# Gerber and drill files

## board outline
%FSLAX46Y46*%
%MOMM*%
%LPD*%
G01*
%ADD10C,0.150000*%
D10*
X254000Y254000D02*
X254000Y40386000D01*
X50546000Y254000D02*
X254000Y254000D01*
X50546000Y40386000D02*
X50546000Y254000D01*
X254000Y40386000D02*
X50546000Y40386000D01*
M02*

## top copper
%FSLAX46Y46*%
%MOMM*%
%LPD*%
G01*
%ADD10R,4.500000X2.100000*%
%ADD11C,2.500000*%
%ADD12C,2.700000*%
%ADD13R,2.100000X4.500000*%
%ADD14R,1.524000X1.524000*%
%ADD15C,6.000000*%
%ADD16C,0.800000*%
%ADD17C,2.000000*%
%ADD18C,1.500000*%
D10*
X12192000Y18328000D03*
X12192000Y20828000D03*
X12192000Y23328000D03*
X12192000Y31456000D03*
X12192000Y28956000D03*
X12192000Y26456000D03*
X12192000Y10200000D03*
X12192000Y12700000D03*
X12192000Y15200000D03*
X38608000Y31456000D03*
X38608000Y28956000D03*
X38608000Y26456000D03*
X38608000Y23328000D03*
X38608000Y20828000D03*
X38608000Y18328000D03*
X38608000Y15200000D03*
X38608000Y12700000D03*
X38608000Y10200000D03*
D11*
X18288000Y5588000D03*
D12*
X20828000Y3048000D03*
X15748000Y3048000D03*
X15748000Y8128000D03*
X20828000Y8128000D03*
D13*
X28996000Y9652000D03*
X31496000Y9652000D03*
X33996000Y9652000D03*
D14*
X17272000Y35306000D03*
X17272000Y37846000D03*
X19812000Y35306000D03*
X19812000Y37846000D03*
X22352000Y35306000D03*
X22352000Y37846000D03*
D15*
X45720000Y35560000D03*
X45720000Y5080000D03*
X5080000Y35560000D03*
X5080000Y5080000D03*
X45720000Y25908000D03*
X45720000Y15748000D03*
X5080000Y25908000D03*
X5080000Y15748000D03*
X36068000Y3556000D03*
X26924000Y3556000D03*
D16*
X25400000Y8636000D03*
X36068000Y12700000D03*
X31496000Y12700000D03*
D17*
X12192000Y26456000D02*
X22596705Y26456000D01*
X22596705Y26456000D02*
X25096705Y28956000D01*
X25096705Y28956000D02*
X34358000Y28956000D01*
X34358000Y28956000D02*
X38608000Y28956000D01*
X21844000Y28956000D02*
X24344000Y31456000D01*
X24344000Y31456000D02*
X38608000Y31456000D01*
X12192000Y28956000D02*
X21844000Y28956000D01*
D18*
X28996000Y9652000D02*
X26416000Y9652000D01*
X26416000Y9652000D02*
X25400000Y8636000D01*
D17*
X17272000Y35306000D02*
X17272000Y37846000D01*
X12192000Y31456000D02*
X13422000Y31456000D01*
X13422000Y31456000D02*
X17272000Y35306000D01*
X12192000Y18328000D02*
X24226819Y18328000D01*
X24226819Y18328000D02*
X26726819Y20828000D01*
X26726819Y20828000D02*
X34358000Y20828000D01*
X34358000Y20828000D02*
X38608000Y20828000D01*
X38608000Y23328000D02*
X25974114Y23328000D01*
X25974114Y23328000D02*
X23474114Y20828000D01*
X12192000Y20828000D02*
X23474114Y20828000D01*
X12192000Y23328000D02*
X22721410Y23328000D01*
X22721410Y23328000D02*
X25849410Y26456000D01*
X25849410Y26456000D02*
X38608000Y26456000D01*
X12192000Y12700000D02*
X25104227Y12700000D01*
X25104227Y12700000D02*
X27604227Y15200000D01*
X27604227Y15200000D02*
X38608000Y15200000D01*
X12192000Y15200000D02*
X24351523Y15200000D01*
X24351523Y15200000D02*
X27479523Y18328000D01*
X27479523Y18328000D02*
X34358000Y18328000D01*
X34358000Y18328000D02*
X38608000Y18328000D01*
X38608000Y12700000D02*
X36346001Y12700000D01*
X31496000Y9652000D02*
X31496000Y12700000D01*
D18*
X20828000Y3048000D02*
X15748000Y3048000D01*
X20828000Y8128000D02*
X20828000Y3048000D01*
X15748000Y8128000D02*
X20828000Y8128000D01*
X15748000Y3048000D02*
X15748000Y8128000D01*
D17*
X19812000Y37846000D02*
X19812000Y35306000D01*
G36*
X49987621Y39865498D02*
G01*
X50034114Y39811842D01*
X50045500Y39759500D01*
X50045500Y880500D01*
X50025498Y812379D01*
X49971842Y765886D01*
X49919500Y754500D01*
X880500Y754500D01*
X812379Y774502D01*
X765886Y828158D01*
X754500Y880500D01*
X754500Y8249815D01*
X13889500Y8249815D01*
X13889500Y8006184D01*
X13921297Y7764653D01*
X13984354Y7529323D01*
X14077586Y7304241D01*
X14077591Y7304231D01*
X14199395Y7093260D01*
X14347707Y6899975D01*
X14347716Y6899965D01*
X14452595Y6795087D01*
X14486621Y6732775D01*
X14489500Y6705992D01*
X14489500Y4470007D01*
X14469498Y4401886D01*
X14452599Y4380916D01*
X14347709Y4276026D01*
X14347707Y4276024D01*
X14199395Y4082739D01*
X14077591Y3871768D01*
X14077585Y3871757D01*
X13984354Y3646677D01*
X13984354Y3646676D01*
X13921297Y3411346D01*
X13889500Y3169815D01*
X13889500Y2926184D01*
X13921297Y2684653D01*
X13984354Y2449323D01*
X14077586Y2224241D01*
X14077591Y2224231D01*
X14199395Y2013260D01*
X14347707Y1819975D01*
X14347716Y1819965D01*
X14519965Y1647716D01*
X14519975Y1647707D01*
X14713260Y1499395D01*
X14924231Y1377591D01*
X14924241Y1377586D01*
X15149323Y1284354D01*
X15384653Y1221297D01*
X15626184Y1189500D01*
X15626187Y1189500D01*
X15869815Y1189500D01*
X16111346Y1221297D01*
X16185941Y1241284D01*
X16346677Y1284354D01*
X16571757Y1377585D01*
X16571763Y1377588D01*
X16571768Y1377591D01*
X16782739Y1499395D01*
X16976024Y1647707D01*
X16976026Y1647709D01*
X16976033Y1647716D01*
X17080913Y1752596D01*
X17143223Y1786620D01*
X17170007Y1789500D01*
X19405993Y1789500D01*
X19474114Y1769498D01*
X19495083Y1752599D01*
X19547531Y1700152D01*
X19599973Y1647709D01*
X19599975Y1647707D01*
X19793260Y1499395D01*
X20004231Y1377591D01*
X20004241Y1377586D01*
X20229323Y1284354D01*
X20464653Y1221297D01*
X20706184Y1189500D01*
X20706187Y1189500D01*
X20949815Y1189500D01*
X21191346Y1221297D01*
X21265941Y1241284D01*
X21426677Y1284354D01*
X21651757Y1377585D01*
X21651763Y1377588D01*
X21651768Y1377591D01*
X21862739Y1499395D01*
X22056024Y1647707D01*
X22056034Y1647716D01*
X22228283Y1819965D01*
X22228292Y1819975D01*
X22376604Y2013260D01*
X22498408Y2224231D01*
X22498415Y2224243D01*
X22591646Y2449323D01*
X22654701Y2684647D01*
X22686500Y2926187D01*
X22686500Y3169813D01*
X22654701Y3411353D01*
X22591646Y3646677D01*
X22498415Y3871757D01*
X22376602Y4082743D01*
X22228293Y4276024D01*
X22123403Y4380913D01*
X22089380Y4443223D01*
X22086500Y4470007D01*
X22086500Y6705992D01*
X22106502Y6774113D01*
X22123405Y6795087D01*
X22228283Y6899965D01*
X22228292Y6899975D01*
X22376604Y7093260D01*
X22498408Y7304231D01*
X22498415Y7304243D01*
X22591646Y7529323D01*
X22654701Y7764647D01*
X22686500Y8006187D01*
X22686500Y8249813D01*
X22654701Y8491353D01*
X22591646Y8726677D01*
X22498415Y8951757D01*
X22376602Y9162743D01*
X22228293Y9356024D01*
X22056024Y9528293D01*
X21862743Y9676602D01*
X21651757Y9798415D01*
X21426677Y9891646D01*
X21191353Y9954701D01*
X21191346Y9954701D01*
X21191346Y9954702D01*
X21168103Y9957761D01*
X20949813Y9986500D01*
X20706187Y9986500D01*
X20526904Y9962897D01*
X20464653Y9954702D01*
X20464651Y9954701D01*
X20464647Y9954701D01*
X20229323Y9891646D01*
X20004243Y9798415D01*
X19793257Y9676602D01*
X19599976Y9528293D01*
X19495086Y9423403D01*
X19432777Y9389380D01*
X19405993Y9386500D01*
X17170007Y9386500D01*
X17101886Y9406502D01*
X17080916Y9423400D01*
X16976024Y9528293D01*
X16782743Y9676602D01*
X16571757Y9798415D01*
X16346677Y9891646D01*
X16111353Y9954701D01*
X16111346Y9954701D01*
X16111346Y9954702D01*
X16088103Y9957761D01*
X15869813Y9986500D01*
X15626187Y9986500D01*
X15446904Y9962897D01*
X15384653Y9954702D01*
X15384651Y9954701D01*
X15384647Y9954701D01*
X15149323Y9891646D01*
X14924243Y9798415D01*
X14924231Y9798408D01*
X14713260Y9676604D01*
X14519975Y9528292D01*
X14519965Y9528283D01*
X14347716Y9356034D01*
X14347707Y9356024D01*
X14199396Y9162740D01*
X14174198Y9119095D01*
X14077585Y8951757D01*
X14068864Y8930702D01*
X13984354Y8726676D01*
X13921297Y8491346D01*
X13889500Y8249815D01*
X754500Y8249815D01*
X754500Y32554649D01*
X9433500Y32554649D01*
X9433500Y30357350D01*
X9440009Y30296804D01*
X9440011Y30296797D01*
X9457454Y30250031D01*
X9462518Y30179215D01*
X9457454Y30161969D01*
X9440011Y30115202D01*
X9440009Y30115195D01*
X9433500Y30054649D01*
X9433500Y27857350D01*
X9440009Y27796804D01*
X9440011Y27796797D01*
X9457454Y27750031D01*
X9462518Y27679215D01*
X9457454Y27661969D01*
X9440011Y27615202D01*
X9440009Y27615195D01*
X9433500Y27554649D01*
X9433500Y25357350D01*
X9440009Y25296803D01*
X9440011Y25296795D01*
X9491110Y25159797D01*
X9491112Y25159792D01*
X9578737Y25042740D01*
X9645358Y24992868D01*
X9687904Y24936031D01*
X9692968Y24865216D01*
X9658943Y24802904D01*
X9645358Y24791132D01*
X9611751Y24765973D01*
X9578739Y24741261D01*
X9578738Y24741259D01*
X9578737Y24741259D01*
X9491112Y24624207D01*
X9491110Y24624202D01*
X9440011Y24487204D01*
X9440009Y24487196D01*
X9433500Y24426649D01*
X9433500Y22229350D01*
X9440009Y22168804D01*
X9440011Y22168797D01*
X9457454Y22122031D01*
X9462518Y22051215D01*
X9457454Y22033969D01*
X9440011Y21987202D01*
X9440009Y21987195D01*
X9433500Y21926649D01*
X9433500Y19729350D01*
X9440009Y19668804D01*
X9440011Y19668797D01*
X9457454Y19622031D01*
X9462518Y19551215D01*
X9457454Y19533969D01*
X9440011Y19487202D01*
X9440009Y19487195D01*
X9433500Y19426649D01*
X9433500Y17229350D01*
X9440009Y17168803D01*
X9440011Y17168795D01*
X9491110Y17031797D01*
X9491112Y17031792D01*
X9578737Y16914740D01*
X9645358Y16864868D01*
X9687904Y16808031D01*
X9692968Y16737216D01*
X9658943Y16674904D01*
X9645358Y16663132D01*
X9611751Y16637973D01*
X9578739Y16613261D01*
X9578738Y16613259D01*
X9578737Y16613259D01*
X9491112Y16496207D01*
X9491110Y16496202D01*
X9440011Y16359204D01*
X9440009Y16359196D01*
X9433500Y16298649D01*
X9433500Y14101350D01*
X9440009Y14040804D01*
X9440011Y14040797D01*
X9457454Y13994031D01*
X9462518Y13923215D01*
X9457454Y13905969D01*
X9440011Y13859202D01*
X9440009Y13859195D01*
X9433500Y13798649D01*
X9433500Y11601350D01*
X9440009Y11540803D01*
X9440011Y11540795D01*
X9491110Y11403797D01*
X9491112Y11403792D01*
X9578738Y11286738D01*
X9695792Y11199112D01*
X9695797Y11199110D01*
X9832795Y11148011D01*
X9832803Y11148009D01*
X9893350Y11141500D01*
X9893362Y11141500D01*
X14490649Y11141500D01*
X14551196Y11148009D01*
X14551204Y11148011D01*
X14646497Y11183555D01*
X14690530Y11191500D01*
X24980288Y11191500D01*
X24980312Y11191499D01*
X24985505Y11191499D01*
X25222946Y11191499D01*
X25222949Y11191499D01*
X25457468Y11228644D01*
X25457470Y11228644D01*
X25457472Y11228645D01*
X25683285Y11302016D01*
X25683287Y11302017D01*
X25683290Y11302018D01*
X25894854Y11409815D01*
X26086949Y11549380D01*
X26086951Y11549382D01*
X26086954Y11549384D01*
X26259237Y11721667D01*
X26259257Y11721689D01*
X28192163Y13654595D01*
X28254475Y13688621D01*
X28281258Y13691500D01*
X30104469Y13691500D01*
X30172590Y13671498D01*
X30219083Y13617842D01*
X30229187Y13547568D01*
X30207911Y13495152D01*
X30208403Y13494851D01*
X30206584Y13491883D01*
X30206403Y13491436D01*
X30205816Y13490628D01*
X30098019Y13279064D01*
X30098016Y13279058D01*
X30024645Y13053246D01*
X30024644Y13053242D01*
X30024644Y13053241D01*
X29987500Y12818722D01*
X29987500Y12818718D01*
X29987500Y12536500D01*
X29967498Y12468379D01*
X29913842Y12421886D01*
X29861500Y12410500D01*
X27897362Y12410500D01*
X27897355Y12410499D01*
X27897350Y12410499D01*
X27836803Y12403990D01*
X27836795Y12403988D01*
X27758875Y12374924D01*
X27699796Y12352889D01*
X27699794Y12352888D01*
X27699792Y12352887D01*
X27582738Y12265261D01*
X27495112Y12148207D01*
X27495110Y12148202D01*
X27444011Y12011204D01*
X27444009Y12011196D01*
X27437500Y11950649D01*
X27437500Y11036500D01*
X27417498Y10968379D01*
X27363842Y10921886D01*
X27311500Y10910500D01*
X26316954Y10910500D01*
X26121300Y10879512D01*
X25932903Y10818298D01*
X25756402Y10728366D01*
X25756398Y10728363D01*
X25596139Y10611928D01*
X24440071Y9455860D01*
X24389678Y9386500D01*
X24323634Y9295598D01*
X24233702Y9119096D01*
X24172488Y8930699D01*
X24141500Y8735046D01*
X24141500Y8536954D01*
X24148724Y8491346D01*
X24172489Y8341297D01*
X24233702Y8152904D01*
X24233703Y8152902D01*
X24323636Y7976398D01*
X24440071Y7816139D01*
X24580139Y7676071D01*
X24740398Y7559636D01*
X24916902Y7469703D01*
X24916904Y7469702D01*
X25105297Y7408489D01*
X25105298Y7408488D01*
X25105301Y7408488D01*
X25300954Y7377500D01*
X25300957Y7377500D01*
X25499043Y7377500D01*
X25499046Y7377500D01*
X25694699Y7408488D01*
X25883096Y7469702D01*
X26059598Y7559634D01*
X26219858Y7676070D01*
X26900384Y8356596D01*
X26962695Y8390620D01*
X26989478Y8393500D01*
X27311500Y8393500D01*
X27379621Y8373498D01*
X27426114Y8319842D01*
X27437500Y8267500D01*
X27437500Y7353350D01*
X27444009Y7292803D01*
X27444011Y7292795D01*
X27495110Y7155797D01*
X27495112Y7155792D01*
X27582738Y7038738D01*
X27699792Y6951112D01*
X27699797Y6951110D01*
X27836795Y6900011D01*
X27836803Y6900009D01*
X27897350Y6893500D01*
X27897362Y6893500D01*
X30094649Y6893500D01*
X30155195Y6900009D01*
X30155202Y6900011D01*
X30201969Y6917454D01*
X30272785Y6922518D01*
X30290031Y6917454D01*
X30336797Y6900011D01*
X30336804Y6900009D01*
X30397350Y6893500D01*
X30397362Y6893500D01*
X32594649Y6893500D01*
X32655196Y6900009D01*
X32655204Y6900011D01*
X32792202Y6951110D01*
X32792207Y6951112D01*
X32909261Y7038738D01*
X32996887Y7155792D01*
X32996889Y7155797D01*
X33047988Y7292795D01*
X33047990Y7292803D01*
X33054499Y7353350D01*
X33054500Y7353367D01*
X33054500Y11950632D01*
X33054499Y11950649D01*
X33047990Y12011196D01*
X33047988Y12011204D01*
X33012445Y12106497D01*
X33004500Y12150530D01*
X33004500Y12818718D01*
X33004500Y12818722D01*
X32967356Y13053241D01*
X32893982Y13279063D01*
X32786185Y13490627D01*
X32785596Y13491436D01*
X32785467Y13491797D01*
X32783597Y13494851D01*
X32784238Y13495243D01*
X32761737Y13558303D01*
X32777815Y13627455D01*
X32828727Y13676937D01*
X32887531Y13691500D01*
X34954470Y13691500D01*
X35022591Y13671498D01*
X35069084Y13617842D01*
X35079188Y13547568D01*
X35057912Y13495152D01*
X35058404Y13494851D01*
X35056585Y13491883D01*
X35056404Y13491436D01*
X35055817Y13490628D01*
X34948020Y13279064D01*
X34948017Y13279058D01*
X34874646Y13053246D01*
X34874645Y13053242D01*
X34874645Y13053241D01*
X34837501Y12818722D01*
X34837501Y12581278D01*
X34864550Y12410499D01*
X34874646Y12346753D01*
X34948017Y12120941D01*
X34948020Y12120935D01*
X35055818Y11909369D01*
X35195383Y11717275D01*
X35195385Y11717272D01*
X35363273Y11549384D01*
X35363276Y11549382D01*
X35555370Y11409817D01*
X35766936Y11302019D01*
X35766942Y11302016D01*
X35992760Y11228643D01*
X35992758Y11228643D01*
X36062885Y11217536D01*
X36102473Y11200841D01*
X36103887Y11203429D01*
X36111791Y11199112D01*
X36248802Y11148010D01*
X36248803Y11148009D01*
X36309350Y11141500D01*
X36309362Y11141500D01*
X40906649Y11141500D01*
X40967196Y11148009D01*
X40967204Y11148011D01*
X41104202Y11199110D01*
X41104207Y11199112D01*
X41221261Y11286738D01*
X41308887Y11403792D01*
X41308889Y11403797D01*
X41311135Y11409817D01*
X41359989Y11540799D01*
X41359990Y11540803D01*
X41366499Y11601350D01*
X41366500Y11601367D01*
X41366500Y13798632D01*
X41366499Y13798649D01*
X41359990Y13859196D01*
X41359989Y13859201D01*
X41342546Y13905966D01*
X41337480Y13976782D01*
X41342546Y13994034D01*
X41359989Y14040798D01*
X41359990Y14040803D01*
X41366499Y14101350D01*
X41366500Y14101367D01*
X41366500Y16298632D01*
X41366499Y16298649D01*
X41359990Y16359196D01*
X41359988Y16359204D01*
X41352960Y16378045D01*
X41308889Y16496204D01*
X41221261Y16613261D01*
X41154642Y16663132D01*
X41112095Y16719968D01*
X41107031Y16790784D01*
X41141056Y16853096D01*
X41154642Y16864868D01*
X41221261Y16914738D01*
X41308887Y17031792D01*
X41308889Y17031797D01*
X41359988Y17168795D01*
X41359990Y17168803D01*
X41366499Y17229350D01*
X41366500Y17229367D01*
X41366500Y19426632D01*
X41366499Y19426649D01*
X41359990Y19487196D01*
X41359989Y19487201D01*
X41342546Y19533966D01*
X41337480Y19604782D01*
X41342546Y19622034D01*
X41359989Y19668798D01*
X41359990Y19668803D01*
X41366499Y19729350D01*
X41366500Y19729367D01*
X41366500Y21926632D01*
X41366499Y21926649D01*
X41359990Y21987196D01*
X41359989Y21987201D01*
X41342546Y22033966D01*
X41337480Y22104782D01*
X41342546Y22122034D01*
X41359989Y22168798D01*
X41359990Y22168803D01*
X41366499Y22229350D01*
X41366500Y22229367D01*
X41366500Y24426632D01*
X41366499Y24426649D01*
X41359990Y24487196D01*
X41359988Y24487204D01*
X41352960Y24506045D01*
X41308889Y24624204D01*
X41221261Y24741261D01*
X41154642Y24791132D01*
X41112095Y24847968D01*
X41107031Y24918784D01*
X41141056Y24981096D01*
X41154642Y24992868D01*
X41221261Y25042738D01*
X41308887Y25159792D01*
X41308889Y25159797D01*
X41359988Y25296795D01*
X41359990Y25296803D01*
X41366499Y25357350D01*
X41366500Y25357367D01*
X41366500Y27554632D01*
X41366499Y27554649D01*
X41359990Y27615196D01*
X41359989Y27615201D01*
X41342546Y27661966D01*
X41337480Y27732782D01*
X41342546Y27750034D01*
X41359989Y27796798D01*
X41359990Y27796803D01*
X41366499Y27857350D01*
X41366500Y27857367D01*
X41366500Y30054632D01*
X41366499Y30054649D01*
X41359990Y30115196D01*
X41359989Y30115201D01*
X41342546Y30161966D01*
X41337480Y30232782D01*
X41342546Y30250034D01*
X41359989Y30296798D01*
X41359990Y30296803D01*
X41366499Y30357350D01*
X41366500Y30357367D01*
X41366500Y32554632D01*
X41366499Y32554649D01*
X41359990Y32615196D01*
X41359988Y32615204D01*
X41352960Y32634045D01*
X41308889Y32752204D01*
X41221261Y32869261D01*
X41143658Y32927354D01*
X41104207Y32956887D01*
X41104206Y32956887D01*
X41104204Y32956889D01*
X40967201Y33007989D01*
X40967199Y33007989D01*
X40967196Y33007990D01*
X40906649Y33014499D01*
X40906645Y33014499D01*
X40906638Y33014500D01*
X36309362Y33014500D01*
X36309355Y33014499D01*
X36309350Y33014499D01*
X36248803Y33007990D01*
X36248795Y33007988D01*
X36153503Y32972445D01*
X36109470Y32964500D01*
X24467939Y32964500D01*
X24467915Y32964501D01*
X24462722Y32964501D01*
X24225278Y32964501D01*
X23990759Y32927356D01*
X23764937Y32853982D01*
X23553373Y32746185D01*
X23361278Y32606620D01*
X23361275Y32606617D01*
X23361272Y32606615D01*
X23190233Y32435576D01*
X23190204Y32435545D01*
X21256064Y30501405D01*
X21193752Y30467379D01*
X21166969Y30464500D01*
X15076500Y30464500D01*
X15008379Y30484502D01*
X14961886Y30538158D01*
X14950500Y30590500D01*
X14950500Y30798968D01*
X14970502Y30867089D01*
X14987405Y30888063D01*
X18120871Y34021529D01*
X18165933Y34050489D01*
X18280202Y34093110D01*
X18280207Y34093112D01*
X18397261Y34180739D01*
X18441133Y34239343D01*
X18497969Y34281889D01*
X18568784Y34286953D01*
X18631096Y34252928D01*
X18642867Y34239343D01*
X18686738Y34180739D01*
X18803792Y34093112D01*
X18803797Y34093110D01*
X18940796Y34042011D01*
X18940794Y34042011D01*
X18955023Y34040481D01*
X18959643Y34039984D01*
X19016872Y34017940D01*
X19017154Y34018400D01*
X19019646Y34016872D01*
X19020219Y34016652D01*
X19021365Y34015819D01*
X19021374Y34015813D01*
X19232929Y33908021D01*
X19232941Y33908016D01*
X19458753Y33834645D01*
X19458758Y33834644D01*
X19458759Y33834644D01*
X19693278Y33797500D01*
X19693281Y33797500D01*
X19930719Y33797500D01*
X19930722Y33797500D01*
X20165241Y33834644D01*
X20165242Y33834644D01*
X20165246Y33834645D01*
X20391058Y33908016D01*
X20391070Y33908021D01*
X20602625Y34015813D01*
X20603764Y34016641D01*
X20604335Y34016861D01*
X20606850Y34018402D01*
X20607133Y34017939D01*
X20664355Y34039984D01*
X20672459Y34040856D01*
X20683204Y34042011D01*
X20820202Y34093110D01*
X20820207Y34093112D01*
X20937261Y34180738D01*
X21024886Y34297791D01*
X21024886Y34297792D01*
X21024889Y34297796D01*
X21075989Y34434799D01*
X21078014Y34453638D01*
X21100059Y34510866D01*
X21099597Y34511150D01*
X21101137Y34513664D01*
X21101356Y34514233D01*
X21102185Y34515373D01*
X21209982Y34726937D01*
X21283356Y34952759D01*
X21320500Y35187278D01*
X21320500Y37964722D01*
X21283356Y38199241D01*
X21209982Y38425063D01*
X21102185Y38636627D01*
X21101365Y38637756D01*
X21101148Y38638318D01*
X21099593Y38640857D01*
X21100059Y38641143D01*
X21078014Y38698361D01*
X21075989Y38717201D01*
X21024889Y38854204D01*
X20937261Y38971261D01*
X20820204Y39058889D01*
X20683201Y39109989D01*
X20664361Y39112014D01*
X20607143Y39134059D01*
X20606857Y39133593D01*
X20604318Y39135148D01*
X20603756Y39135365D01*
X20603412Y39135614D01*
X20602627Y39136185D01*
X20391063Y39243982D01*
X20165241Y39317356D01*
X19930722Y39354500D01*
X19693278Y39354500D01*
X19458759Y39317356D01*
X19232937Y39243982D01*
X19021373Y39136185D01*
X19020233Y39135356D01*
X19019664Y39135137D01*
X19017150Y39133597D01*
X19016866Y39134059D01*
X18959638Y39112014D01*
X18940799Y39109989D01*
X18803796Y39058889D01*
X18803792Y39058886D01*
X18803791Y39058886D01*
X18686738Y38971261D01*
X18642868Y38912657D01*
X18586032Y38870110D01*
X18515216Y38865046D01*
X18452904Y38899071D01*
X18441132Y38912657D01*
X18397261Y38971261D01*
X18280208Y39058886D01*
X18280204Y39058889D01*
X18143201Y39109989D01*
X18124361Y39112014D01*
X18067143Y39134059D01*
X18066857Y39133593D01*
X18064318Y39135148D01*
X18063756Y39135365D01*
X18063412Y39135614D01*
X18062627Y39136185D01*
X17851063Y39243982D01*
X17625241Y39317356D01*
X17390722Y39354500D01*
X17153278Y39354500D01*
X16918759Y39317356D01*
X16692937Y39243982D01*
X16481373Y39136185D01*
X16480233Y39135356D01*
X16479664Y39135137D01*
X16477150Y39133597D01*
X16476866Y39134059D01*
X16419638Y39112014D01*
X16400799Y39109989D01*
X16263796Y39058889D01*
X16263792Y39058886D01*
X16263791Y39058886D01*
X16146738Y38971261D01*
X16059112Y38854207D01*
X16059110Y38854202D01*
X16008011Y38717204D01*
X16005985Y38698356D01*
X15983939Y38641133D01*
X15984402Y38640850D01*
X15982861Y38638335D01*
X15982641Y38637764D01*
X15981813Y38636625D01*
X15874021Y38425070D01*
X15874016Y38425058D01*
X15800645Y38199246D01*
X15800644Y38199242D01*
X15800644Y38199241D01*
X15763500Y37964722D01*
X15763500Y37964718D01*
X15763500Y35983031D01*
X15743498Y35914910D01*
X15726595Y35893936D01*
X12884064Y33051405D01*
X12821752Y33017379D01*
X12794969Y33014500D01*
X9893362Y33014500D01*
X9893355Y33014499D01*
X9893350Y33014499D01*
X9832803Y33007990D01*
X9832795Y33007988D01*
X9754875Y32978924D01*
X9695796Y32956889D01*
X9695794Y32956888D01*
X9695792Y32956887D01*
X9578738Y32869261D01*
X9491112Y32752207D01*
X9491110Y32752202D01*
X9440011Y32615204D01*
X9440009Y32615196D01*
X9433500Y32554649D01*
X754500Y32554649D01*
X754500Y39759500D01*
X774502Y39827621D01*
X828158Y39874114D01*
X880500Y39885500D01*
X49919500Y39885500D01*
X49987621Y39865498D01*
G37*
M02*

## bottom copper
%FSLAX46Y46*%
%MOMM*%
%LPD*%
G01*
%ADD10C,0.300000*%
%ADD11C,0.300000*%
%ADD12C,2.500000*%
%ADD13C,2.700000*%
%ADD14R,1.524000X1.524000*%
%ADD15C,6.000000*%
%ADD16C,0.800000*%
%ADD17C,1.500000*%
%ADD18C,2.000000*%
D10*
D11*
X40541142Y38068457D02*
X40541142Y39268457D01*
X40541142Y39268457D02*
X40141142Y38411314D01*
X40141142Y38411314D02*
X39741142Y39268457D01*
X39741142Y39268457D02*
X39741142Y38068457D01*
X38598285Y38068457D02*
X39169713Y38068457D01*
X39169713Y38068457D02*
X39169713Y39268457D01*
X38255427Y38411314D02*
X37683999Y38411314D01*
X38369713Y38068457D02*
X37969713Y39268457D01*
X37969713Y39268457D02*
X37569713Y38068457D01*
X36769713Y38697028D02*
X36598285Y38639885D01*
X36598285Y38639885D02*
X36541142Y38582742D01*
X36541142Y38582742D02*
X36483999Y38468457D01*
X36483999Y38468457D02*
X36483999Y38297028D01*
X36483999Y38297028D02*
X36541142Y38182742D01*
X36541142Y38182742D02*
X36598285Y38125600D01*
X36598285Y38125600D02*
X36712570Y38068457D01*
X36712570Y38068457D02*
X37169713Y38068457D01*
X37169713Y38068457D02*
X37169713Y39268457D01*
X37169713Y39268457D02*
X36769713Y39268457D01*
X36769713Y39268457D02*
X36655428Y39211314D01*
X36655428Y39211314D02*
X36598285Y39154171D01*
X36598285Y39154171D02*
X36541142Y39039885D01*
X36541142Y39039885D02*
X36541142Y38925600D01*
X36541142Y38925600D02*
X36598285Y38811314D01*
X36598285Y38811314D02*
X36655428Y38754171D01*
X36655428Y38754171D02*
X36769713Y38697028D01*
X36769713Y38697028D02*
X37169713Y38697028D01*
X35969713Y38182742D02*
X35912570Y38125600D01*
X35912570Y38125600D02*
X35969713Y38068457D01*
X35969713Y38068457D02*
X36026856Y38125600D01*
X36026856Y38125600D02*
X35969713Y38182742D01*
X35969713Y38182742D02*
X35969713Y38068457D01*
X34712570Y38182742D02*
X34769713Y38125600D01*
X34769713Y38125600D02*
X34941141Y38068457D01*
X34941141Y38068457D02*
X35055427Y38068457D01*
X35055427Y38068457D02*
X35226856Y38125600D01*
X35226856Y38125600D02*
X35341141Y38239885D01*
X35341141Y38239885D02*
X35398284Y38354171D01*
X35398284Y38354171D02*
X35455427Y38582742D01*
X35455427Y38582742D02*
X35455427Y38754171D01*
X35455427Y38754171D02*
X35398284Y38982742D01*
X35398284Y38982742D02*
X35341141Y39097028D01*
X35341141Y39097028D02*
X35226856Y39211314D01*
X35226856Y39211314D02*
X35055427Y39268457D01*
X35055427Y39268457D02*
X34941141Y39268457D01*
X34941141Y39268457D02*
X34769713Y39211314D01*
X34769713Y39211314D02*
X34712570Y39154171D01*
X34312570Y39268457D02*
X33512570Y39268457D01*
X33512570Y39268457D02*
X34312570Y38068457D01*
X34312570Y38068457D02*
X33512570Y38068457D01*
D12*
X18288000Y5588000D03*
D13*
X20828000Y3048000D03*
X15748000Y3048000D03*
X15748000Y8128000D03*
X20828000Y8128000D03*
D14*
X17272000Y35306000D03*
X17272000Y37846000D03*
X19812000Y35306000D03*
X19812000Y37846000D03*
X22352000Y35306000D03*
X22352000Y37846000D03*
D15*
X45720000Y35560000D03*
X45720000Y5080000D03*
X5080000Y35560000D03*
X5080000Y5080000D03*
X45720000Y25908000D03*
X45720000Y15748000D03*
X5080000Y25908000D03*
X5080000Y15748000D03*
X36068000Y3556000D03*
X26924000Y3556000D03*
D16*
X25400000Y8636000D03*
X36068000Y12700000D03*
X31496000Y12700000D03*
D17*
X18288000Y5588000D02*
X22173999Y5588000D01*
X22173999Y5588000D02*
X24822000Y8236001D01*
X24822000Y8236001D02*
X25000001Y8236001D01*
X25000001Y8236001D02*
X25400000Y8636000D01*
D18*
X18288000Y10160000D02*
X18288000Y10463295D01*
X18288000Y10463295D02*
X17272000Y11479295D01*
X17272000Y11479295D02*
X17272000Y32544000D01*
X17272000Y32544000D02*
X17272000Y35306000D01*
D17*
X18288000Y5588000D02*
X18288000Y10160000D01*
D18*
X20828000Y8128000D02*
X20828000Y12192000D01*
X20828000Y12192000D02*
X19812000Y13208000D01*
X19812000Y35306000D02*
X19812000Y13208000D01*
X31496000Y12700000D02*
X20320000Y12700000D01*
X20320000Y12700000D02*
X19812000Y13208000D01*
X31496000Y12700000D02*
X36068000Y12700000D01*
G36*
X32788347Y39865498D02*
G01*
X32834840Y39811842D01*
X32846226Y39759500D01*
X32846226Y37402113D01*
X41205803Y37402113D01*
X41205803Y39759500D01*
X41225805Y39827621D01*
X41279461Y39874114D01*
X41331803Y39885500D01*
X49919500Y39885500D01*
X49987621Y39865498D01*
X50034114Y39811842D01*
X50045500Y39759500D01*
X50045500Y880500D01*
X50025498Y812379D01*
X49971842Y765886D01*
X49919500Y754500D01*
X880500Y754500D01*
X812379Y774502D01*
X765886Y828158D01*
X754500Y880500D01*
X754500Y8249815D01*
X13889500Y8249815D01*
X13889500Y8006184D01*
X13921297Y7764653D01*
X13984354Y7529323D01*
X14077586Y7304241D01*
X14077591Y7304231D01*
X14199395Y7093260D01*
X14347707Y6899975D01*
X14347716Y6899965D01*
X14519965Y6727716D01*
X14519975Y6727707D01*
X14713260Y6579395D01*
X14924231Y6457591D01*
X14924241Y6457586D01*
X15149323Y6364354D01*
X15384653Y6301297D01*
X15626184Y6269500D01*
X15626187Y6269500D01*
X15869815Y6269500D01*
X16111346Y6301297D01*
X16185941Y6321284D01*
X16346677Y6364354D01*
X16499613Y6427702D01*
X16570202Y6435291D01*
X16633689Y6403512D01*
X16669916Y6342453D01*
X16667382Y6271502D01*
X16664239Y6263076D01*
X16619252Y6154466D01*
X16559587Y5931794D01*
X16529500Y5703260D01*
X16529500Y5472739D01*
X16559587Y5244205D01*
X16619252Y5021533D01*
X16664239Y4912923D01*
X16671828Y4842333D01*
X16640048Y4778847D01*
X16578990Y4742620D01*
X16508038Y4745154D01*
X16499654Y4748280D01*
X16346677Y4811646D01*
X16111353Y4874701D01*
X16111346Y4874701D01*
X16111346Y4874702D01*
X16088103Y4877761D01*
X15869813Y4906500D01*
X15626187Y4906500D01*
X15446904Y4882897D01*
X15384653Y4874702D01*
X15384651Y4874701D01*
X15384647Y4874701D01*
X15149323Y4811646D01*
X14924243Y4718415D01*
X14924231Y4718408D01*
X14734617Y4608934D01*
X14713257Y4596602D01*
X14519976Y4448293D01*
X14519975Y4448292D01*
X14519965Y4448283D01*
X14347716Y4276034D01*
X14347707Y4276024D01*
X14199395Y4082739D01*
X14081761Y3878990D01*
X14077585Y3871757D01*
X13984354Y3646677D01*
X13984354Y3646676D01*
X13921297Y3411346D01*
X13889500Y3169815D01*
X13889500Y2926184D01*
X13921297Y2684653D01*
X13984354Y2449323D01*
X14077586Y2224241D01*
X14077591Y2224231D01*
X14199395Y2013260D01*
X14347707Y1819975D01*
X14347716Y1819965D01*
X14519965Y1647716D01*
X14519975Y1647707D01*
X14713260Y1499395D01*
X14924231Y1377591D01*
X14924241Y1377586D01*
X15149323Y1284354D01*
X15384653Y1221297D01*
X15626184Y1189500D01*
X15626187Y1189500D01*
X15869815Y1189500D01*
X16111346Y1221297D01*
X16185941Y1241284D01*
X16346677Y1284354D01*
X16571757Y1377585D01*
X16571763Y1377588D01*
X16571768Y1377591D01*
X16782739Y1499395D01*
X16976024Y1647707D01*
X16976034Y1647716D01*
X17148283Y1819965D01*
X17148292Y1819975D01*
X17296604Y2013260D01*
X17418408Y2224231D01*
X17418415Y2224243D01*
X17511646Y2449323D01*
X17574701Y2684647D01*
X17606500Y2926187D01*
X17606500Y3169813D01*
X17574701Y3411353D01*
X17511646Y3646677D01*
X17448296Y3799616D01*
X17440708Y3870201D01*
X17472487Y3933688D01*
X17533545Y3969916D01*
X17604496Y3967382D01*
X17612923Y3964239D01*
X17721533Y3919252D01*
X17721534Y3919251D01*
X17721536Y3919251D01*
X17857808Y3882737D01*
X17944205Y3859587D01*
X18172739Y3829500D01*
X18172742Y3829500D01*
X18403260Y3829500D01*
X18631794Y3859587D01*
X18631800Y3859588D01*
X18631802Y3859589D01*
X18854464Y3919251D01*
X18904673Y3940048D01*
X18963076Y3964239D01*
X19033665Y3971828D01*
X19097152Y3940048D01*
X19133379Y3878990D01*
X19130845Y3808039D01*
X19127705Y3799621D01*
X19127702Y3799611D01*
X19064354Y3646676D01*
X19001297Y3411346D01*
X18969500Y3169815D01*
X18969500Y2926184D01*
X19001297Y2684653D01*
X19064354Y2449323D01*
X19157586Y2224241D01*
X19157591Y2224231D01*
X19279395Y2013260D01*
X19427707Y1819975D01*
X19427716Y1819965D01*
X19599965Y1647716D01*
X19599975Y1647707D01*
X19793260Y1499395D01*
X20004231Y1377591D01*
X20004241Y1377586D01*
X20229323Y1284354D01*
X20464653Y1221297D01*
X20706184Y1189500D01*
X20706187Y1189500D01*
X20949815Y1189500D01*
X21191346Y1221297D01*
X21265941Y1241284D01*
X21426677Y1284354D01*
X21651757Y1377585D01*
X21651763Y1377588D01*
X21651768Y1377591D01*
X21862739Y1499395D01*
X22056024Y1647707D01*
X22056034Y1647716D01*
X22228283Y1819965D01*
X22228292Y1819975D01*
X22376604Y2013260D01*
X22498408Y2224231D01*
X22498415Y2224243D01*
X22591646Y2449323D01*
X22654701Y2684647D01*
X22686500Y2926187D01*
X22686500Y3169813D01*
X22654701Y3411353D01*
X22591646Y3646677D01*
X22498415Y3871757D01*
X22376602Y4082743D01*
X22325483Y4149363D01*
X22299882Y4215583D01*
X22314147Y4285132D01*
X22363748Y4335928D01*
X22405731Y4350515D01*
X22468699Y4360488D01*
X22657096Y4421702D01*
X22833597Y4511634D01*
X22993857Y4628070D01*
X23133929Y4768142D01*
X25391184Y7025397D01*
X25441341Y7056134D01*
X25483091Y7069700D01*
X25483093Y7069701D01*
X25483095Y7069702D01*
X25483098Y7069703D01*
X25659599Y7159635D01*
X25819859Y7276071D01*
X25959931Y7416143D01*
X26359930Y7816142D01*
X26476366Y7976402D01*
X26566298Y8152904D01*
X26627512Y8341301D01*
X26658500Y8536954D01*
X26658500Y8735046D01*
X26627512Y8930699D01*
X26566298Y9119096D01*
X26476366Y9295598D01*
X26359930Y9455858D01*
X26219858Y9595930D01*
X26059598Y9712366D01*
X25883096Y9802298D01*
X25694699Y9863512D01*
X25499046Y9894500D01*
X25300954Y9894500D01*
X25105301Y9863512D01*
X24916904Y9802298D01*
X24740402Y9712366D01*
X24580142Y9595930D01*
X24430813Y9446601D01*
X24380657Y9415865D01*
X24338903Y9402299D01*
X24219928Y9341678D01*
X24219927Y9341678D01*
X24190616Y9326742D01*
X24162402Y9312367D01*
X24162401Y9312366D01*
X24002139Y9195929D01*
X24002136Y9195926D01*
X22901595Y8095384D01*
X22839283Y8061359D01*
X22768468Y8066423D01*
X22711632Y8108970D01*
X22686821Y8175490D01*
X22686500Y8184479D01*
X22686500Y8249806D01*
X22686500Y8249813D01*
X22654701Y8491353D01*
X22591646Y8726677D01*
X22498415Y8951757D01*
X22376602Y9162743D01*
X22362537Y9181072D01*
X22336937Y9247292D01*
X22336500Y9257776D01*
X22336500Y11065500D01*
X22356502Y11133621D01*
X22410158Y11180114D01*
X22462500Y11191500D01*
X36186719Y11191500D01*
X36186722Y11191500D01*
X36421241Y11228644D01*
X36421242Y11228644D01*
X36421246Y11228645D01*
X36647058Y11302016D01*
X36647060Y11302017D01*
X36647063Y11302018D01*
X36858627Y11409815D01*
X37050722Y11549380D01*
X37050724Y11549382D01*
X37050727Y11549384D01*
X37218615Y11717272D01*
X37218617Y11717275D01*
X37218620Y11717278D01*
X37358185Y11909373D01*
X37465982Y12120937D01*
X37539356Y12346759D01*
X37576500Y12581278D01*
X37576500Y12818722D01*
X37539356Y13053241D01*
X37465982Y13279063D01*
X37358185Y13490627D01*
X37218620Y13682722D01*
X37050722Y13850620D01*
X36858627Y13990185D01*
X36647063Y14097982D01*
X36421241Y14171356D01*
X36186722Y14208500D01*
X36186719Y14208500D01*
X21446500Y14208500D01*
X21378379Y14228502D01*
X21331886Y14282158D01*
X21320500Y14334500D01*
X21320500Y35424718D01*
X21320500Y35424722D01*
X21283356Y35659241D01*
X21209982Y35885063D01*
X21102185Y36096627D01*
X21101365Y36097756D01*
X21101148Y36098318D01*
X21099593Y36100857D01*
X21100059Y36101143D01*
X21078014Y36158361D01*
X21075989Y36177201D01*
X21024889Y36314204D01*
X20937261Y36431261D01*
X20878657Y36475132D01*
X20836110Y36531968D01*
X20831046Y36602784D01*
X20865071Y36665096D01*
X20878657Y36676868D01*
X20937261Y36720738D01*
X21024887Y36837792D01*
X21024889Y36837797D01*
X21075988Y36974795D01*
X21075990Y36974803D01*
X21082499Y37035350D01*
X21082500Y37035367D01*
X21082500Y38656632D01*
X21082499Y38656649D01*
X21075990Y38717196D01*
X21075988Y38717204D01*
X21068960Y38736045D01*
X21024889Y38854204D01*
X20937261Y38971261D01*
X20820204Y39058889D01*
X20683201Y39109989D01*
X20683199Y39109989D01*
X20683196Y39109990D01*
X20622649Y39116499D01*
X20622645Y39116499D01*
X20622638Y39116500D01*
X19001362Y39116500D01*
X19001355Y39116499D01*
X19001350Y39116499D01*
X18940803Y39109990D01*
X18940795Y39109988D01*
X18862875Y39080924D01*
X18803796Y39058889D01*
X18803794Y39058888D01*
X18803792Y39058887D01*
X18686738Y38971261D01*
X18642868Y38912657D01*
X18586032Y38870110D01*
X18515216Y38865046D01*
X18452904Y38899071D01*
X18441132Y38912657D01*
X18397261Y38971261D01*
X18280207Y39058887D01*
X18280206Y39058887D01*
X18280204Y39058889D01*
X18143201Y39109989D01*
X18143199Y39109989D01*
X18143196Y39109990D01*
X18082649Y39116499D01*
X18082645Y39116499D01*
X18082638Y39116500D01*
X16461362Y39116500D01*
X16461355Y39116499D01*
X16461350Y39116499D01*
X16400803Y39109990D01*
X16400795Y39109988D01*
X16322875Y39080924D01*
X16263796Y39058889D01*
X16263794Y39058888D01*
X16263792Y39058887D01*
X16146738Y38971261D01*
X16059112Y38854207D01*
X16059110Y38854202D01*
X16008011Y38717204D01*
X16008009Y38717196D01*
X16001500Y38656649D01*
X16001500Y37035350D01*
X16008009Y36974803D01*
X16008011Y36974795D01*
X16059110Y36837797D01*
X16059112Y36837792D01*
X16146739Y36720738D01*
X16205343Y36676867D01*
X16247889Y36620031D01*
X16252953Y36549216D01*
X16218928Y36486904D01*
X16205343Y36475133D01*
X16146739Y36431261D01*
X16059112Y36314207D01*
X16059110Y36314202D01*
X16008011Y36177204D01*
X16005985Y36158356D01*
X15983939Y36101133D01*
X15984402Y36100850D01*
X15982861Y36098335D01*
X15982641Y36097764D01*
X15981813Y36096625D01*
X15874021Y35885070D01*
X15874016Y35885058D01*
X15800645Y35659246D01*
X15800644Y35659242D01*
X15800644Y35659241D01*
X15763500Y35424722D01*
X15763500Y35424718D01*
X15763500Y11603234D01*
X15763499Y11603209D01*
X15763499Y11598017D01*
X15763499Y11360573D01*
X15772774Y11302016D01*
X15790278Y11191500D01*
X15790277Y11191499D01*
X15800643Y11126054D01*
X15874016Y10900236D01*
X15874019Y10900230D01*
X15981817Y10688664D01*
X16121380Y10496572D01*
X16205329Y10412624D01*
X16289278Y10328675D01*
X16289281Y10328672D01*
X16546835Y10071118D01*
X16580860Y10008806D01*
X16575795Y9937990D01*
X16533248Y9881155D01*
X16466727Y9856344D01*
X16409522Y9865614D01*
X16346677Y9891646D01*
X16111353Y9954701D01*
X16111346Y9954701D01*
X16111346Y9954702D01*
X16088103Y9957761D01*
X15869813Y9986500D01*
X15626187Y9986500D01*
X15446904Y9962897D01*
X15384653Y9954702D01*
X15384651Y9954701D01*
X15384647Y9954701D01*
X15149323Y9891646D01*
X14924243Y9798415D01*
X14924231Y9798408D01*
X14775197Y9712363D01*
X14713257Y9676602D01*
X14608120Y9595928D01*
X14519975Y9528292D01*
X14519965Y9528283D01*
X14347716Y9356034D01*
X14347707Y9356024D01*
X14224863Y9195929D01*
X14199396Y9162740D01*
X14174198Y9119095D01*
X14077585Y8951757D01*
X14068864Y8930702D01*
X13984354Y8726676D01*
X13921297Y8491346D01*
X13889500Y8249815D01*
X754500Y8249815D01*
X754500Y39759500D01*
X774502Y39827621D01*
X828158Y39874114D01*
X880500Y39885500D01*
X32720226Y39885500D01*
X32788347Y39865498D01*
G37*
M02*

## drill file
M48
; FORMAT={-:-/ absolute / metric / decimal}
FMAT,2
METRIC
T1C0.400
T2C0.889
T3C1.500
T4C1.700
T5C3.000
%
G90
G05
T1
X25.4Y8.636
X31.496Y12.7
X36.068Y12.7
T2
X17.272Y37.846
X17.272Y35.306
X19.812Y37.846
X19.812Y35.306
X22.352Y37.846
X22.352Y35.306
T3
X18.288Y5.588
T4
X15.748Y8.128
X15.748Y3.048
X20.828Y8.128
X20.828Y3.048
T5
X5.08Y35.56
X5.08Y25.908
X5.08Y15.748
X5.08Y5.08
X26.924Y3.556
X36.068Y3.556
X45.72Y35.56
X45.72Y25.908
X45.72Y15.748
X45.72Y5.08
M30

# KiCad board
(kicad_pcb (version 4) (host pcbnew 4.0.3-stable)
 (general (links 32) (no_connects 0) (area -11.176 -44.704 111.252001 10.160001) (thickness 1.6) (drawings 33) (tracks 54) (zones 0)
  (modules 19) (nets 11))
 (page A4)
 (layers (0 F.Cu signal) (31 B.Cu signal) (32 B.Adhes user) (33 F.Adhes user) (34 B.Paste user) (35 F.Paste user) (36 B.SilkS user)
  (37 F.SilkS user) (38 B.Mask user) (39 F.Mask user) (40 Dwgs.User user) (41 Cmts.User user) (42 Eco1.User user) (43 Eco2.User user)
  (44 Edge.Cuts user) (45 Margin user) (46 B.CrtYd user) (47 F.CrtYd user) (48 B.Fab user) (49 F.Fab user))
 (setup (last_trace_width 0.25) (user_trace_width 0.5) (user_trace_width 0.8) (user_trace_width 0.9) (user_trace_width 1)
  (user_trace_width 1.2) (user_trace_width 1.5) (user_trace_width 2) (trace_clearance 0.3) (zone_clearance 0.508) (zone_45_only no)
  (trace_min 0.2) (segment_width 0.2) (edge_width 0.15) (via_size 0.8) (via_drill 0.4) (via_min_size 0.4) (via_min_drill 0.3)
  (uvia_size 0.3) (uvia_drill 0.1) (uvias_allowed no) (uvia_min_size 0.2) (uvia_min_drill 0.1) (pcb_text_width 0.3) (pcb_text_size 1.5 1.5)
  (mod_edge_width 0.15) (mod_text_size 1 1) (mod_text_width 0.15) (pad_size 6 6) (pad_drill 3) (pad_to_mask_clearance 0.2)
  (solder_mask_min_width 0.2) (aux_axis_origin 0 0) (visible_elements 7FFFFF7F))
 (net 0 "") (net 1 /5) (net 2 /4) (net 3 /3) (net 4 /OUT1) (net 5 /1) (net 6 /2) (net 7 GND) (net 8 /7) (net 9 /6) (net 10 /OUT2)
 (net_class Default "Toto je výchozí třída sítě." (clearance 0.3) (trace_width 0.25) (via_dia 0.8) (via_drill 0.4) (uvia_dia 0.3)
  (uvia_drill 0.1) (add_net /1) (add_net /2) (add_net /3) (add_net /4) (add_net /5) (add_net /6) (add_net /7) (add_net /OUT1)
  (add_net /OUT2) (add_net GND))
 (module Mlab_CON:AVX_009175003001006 (layer F.Cu) (at 12.192 -20.828 90)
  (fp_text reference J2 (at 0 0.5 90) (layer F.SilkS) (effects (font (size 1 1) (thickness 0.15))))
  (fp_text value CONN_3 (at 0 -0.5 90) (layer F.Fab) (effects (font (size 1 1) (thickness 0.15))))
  (pad 1 smd rect (at -2.5 0 90) (size 2.1 4.5) (layers F.Cu F.Paste F.Mask) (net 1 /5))
  (pad 2 smd rect (at 0 0 90) (size 2.1 4.5) (layers F.Cu F.Paste F.Mask) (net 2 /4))
  (pad 3 smd rect (at 2.5 0 90) (size 2.1 4.5) (layers F.Cu F.Paste F.Mask) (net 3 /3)))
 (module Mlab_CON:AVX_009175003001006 (layer F.Cu) (at 12.192 -28.956 270)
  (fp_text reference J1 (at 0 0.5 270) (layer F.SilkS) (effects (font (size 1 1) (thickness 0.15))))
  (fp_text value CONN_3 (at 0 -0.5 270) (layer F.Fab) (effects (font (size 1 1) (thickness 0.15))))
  (pad 1 smd rect (at -2.5 0 270) (size 2.1 4.5) (layers F.Cu F.Paste F.Mask) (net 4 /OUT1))
  (pad 2 smd rect (at 0 0 270) (size 2.1 4.5) (layers F.Cu F.Paste F.Mask) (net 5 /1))
  (pad 3 smd rect (at 2.5 0 270) (size 2.1 4.5) (layers F.Cu F.Paste F.Mask) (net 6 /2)))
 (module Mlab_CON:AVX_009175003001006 (layer F.Cu) (at 12.192 -12.7 90)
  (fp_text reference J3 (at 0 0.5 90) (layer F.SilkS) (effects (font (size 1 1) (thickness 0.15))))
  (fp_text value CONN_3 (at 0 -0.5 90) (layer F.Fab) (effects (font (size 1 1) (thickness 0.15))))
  (pad 1 smd rect (at -2.5 0 90) (size 2.1 4.5) (layers F.Cu F.Paste F.Mask) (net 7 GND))
  (pad 2 smd rect (at 0 0 90) (size 2.1 4.5) (layers F.Cu F.Paste F.Mask) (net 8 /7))
  (pad 3 smd rect (at 2.5 0 90) (size 2.1 4.5) (layers F.Cu F.Paste F.Mask) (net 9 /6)))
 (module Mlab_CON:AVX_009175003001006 (layer F.Cu) (at 38.608 -28.956 270)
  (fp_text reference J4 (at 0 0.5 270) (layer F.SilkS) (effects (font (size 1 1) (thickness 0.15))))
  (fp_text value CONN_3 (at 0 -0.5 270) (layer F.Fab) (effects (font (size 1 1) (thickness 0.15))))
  (pad 1 smd rect (at -2.5 0 270) (size 2.1 4.5) (layers F.Cu F.Paste F.Mask) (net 5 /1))
  (pad 2 smd rect (at 0 0 270) (size 2.1 4.5) (layers F.Cu F.Paste F.Mask) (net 6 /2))
  (pad 3 smd rect (at 2.5 0 270) (size 2.1 4.5) (layers F.Cu F.Paste F.Mask) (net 3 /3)))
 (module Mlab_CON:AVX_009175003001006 (layer F.Cu) (at 38.608 -20.828 270)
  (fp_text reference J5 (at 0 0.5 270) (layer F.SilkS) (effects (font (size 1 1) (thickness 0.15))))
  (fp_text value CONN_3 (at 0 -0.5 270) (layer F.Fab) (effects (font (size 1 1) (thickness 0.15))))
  (pad 1 smd rect (at -2.5 0 270) (size 2.1 4.5) (layers F.Cu F.Paste F.Mask) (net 2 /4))
  (pad 2 smd rect (at 0 0 270) (size 2.1 4.5) (layers F.Cu F.Paste F.Mask) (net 1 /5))
  (pad 3 smd rect (at 2.5 0 270) (size 2.1 4.5) (layers F.Cu F.Paste F.Mask) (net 9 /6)))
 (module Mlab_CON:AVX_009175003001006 (layer F.Cu) (at 38.608 -12.7 270)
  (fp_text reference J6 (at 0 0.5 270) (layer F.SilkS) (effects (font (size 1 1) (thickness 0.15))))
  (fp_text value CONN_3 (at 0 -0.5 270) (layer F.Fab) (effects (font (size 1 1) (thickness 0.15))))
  (pad 1 smd rect (at -2.5 0 270) (size 2.1 4.5) (layers F.Cu F.Paste F.Mask) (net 8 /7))
  (pad 2 smd rect (at 0 0 270) (size 2.1 4.5) (layers F.Cu F.Paste F.Mask) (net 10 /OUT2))
  (pad 3 smd rect (at 2.5 0 270) (size 2.1 4.5) (layers F.Cu F.Paste F.Mask) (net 7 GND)))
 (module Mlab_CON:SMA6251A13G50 (layer F.Cu) (at 18.288 -5.588)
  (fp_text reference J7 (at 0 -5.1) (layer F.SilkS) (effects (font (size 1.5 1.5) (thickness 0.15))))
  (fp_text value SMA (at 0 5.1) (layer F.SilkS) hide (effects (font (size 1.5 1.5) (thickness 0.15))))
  (pad 1 thru_hole circle (at 0 0 180) (size 2.5 2.5) (drill 1.5) (layers *.Cu *.Mask) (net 4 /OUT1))
  (pad 2 thru_hole circle (at 2.54 2.54 180) (size 2.7 2.7) (drill 1.7) (layers *.Cu *.Mask) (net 10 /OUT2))
  (pad 2 thru_hole circle (at -2.54 2.54 180) (size 2.7 2.7) (drill 1.7) (layers *.Cu *.Mask) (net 10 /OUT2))
  (pad 2 thru_hole circle (at -2.54 -2.54 180) (size 2.7 2.7) (drill 1.7) (layers *.Cu *.Mask) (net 10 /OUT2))
  (pad 2 thru_hole circle (at 2.54 -2.54 180) (size 2.7 2.7) (drill 1.7) (layers *.Cu *.Mask) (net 10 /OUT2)))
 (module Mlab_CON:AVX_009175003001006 (layer F.Cu) (at 31.496 -9.652)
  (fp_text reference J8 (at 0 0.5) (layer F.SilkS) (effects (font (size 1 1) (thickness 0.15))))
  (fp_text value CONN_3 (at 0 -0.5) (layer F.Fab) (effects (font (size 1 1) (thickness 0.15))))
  (pad 1 smd rect (at -2.5 0) (size 2.1 4.5) (layers F.Cu F.Paste F.Mask) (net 4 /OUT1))
  (pad 2 smd rect (at 0 0) (size 2.1 4.5) (layers F.Cu F.Paste F.Mask) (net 10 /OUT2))
  (pad 3 smd rect (at 2.5 0) (size 2.1 4.5) (layers F.Cu F.Paste F.Mask) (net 7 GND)))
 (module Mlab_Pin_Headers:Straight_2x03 (layer F.Cu) (at 19.812 -36.576 90)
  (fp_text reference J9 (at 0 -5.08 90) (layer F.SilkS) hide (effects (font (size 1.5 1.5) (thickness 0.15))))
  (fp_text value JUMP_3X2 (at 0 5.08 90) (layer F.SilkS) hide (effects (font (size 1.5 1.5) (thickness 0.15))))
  (pad 1 thru_hole rect (at -1.27 -2.54 90) (size 1.524 1.524) (drill 0.889) (layers *.Cu *.Mask F.SilkS) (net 4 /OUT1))
  (pad 2 thru_hole rect (at 1.27 -2.54 90) (size 1.524 1.524) (drill 0.889) (layers *.Cu *.Mask F.SilkS) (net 4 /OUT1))
  (pad 3 thru_hole rect (at -1.27 0 90) (size 1.524 1.524) (drill 0.889) (layers *.Cu *.Mask F.SilkS) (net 10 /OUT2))
  (pad 4 thru_hole rect (at 1.27 0 90) (size 1.524 1.524) (drill 0.889) (layers *.Cu *.Mask F.SilkS) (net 10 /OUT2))
  (pad 5 thru_hole rect (at -1.27 2.54 90) (size 1.524 1.524) (drill 0.889) (layers *.Cu *.Mask F.SilkS) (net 7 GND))
  (pad 6 thru_hole rect (at 1.27 2.54 90) (size 1.524 1.524) (drill 0.889) (layers *.Cu *.Mask F.SilkS) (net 7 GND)))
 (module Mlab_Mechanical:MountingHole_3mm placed (layer F.Cu) (at 45.72 -35.56)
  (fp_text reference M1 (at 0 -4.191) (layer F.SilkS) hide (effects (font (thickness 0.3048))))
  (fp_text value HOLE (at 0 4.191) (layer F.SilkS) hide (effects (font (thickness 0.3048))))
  (pad 1 thru_hole circle (at 0 0) (size 6 6) (drill 3) (layers *.Cu *.Adhes *.Mask) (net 7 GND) (clearance 1) (zone_connect 2)))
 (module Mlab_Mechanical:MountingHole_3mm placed (layer F.Cu) (at 45.72 -5.08)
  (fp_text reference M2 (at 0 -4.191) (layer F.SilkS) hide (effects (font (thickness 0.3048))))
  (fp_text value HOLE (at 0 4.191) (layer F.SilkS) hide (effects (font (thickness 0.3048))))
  (pad 1 thru_hole circle (at 0 0) (size 6 6) (drill 3) (layers *.Cu *.Adhes *.Mask) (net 7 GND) (clearance 1) (zone_connect 2)))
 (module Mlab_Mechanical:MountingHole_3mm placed (layer F.Cu) (at 5.08 -35.56)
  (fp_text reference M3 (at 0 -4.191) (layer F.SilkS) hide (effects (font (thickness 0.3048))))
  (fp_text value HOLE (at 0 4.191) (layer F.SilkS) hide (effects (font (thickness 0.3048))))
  (pad 1 thru_hole circle (at 0 0) (size 6 6) (drill 3) (layers *.Cu *.Adhes *.Mask) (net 7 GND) (clearance 1) (zone_connect 2)))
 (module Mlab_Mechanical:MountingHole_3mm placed (layer F.Cu) (at 5.08 -5.08)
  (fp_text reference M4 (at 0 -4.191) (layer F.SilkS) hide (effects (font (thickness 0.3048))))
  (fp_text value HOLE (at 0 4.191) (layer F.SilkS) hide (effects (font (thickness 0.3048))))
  (pad 1 thru_hole circle (at 0 0) (size 6 6) (drill 3) (layers *.Cu *.Adhes *.Mask) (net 7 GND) (clearance 1) (zone_connect 2)))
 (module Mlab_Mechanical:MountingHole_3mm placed (layer F.Cu) (at 45.72 -25.908)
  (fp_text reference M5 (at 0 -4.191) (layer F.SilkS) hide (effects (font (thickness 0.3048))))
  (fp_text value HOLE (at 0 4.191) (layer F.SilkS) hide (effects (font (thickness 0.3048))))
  (pad 1 thru_hole circle (at 0 0) (size 6 6) (drill 3) (layers *.Cu *.Adhes *.Mask) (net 7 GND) (clearance 1) (zone_connect 2)))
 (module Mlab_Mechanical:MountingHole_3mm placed (layer F.Cu) (at 45.72 -15.748)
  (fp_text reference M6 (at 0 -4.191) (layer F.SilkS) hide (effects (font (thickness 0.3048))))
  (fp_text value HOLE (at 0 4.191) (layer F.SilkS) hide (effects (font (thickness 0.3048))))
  (pad 1 thru_hole circle (at 0 0) (size 6 6) (drill 3) (layers *.Cu *.Adhes *.Mask) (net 7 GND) (clearance 1) (zone_connect 2)))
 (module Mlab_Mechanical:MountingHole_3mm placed (layer F.Cu) (at 5.08 -25.908)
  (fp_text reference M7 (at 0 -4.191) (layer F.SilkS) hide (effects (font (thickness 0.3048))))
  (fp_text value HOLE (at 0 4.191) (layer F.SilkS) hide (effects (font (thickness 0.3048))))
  (pad 1 thru_hole circle (at 0 0) (size 6 6) (drill 3) (layers *.Cu *.Adhes *.Mask) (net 7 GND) (clearance 1) (zone_connect 2)))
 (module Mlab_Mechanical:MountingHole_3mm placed (layer F.Cu) (at 5.08 -15.748)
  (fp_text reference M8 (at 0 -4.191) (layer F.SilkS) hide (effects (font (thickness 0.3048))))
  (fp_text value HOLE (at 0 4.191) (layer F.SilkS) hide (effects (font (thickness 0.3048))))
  (pad 1 thru_hole circle (at 0 0) (size 6 6) (drill 3) (layers *.Cu *.Adhes *.Mask) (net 7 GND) (clearance 1) (zone_connect 2)))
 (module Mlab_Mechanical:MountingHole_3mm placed (layer F.Cu) (at 36.068 -3.556)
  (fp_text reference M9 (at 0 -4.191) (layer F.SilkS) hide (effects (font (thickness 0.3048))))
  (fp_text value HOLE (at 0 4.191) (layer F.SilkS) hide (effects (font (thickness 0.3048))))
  (pad 1 thru_hole circle (at 0 0) (size 6 6) (drill 3) (layers *.Cu *.Adhes *.Mask) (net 7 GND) (clearance 1) (zone_connect 2)))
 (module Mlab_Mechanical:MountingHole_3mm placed (layer F.Cu) (at 26.924 -3.556)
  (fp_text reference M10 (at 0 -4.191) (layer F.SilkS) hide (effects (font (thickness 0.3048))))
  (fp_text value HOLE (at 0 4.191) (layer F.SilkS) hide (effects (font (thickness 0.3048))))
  (pad 1 thru_hole circle (at 0 0) (size 6 6) (drill 3) (layers *.Cu *.Adhes *.Mask) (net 7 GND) (clearance 1) (zone_connect 2)))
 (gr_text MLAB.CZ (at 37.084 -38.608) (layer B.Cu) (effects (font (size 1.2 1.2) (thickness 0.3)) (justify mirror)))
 (gr_line (start 0.254 -0.254) (end 0.254 -40.386) (angle 90) (layer Edge.Cuts) (width 0.15))
 (gr_line (start 50.546 -0.254) (end 0.254 -0.254) (angle 90) (layer Edge.Cuts) (width 0.15))
 (gr_line (start 50.546 -40.386) (end 50.546 -0.254) (angle 90) (layer Edge.Cuts) (width 0.15))
 (gr_line (start 0.254 -40.386) (end 50.546 -40.386) (angle 90) (layer Edge.Cuts) (width 0.15))
 (segment (start 12.192 -26.456) (end 22.596705 -26.456) (width 2) (layer F.Cu) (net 6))
 (segment (start 22.596705 -26.456) (end 25.096705 -28.956) (width 2) (layer F.Cu) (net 6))
 (segment (start 25.096705 -28.956) (end 34.358 -28.956) (width 2) (layer F.Cu) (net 6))
 (segment (start 34.358 -28.956) (end 38.608 -28.956) (width 2) (layer F.Cu) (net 6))
 (segment (start 21.844 -28.956) (end 24.344 -31.456) (width 2) (layer F.Cu) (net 5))
 (segment (start 24.344 -31.456) (end 38.608 -31.456) (width 2) (layer F.Cu) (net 5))
 (segment (start 12.192 -28.956) (end 21.844 -28.956) (width 2) (layer F.Cu) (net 5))
 (segment (start 18.288 -5.588) (end 22.173999 -5.588) (width 1.5) (layer B.Cu) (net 4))
 (segment (start 22.173999 -5.588) (end 24.822 -8.236001) (width 1.5) (layer B.Cu) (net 4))
 (segment (start 24.822 -8.236001) (end 25.000001 -8.236001) (width 1.5) (layer B.Cu) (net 4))
 (segment (start 25.000001 -8.236001) (end 25.4 -8.636) (width 1.5) (layer B.Cu) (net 4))
 (segment (start 28.996 -9.652) (end 26.416 -9.652) (width 1.5) (layer F.Cu) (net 4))
 (segment (start 26.416 -9.652) (end 25.4 -8.636) (width 1.5) (layer F.Cu) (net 4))
 (via (at 25.4 -8.636) (size 0.8) (drill 0.4) (layers F.Cu B.Cu) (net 4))
 (segment (start 18.288 -10.16) (end 18.288 -10.463295) (width 2) (layer B.Cu) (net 4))
 (segment (start 18.288 -10.463295) (end 17.272 -11.479295) (width 2) (layer B.Cu) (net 4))
 (segment (start 17.272 -11.479295) (end 17.272 -32.544) (width 2) (layer B.Cu) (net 4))
 (segment (start 17.272 -32.544) (end 17.272 -35.306) (width 2) (layer B.Cu) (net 4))
 (segment (start 18.288 -5.588) (end 18.288 -10.16) (width 1.5) (layer B.Cu) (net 4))
 (segment (start 17.272 -35.306) (end 17.272 -37.846) (width 2) (layer F.Cu) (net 4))
 (segment (start 12.192 -31.456) (end 13.422 -31.456) (width 2) (layer F.Cu) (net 4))
 (segment (start 13.422 -31.456) (end 17.272 -35.306) (width 2) (layer F.Cu) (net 4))
 (segment (start 12.192 -18.328) (end 24.226819 -18.328) (width 2) (layer F.Cu) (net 1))
 (segment (start 24.226819 -18.328) (end 26.726819 -20.828) (width 2) (layer F.Cu) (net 1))
 (segment (start 26.726819 -20.828) (end 34.358 -20.828) (width 2) (layer F.Cu) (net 1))
 (segment (start 34.358 -20.828) (end 38.608 -20.828) (width 2) (layer F.Cu) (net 1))
 (segment (start 38.608 -23.328) (end 25.974114 -23.328) (width 2) (layer F.Cu) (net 2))
 (segment (start 25.974114 -23.328) (end 23.474114 -20.828) (width 2) (layer F.Cu) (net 2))
 (segment (start 12.192 -20.828) (end 23.474114 -20.828) (width 2) (layer F.Cu) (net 2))
 (segment (start 12.192 -23.328) (end 22.72141 -23.328) (width 2) (layer F.Cu) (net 3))
 (segment (start 22.72141 -23.328) (end 25.84941 -26.456) (width 2) (layer F.Cu) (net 3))
 (segment (start 25.84941 -26.456) (end 38.608 -26.456) (width 2) (layer F.Cu) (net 3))
 (segment (start 12.192 -12.7) (end 25.104227 -12.7) (width 2) (layer F.Cu) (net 8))
 (segment (start 25.104227 -12.7) (end 27.604227 -15.2) (width 2) (layer F.Cu) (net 8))
 (segment (start 27.604227 -15.2) (end 38.608 -15.2) (width 2) (layer F.Cu) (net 8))
 (segment (start 12.192 -15.2) (end 24.351523 -15.2) (width 2) (layer F.Cu) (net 9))
 (segment (start 24.351523 -15.2) (end 27.479523 -18.328) (width 2) (layer F.Cu) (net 9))
 (segment (start 27.479523 -18.328) (end 34.358 -18.328) (width 2) (layer F.Cu) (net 9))
 (segment (start 34.358 -18.328) (end 38.608 -18.328) (width 2) (layer F.Cu) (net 9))
 (segment (start 20.828 -8.128) (end 20.828 -12.192) (width 2) (layer B.Cu) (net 10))
 (segment (start 20.828 -12.192) (end 19.812 -13.208) (width 2) (layer B.Cu) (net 10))
 (segment (start 19.812 -35.306) (end 19.812 -13.208) (width 2) (layer B.Cu) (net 10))
 (segment (start 31.496 -12.7) (end 20.32 -12.7) (width 2) (layer B.Cu) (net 10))
 (segment (start 20.32 -12.7) (end 19.812 -13.208) (width 2) (layer B.Cu) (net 10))
 (segment (start 38.608 -12.7) (end 36.346001 -12.7) (width 2) (layer F.Cu) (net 10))
 (segment (start 31.496 -12.7) (end 36.068 -12.7) (width 2) (layer B.Cu) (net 10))
 (via (at 36.068 -12.7) (size 0.8) (drill 0.4) (layers F.Cu B.Cu) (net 10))
 (segment (start 31.496 -9.652) (end 31.496 -12.7) (width 2) (layer F.Cu) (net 10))
 (via (at 31.496 -12.7) (size 0.8) (drill 0.4) (layers F.Cu B.Cu) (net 10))
 (segment (start 20.828 -3.048) (end 15.748 -3.048) (width 1.5) (layer F.Cu) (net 10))
 (segment (start 20.828 -8.128) (end 20.828 -3.048) (width 1.5) (layer F.Cu) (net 10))
 (segment (start 15.748 -8.128) (end 20.828 -8.128) (width 1.5) (layer F.Cu) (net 10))
 (segment (start 15.748 -3.048) (end 15.748 -8.128) (width 1.5) (layer F.Cu) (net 10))
 (segment (start 19.812 -37.846) (end 19.812 -35.306) (width 2) (layer F.Cu) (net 10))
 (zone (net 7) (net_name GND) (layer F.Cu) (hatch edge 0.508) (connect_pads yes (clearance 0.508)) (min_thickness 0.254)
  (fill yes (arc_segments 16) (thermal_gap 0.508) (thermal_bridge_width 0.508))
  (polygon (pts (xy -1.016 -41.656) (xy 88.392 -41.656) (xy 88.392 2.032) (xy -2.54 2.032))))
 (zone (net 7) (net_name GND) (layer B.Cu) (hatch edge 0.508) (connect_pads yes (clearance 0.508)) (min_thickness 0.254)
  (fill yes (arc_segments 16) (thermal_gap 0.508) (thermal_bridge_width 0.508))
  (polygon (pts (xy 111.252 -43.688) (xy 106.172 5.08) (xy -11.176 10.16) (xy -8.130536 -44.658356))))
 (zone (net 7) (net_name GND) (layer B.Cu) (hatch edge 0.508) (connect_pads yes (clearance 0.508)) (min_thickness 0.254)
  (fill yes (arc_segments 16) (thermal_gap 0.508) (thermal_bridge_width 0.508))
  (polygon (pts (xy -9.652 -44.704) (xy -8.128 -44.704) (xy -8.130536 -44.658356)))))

